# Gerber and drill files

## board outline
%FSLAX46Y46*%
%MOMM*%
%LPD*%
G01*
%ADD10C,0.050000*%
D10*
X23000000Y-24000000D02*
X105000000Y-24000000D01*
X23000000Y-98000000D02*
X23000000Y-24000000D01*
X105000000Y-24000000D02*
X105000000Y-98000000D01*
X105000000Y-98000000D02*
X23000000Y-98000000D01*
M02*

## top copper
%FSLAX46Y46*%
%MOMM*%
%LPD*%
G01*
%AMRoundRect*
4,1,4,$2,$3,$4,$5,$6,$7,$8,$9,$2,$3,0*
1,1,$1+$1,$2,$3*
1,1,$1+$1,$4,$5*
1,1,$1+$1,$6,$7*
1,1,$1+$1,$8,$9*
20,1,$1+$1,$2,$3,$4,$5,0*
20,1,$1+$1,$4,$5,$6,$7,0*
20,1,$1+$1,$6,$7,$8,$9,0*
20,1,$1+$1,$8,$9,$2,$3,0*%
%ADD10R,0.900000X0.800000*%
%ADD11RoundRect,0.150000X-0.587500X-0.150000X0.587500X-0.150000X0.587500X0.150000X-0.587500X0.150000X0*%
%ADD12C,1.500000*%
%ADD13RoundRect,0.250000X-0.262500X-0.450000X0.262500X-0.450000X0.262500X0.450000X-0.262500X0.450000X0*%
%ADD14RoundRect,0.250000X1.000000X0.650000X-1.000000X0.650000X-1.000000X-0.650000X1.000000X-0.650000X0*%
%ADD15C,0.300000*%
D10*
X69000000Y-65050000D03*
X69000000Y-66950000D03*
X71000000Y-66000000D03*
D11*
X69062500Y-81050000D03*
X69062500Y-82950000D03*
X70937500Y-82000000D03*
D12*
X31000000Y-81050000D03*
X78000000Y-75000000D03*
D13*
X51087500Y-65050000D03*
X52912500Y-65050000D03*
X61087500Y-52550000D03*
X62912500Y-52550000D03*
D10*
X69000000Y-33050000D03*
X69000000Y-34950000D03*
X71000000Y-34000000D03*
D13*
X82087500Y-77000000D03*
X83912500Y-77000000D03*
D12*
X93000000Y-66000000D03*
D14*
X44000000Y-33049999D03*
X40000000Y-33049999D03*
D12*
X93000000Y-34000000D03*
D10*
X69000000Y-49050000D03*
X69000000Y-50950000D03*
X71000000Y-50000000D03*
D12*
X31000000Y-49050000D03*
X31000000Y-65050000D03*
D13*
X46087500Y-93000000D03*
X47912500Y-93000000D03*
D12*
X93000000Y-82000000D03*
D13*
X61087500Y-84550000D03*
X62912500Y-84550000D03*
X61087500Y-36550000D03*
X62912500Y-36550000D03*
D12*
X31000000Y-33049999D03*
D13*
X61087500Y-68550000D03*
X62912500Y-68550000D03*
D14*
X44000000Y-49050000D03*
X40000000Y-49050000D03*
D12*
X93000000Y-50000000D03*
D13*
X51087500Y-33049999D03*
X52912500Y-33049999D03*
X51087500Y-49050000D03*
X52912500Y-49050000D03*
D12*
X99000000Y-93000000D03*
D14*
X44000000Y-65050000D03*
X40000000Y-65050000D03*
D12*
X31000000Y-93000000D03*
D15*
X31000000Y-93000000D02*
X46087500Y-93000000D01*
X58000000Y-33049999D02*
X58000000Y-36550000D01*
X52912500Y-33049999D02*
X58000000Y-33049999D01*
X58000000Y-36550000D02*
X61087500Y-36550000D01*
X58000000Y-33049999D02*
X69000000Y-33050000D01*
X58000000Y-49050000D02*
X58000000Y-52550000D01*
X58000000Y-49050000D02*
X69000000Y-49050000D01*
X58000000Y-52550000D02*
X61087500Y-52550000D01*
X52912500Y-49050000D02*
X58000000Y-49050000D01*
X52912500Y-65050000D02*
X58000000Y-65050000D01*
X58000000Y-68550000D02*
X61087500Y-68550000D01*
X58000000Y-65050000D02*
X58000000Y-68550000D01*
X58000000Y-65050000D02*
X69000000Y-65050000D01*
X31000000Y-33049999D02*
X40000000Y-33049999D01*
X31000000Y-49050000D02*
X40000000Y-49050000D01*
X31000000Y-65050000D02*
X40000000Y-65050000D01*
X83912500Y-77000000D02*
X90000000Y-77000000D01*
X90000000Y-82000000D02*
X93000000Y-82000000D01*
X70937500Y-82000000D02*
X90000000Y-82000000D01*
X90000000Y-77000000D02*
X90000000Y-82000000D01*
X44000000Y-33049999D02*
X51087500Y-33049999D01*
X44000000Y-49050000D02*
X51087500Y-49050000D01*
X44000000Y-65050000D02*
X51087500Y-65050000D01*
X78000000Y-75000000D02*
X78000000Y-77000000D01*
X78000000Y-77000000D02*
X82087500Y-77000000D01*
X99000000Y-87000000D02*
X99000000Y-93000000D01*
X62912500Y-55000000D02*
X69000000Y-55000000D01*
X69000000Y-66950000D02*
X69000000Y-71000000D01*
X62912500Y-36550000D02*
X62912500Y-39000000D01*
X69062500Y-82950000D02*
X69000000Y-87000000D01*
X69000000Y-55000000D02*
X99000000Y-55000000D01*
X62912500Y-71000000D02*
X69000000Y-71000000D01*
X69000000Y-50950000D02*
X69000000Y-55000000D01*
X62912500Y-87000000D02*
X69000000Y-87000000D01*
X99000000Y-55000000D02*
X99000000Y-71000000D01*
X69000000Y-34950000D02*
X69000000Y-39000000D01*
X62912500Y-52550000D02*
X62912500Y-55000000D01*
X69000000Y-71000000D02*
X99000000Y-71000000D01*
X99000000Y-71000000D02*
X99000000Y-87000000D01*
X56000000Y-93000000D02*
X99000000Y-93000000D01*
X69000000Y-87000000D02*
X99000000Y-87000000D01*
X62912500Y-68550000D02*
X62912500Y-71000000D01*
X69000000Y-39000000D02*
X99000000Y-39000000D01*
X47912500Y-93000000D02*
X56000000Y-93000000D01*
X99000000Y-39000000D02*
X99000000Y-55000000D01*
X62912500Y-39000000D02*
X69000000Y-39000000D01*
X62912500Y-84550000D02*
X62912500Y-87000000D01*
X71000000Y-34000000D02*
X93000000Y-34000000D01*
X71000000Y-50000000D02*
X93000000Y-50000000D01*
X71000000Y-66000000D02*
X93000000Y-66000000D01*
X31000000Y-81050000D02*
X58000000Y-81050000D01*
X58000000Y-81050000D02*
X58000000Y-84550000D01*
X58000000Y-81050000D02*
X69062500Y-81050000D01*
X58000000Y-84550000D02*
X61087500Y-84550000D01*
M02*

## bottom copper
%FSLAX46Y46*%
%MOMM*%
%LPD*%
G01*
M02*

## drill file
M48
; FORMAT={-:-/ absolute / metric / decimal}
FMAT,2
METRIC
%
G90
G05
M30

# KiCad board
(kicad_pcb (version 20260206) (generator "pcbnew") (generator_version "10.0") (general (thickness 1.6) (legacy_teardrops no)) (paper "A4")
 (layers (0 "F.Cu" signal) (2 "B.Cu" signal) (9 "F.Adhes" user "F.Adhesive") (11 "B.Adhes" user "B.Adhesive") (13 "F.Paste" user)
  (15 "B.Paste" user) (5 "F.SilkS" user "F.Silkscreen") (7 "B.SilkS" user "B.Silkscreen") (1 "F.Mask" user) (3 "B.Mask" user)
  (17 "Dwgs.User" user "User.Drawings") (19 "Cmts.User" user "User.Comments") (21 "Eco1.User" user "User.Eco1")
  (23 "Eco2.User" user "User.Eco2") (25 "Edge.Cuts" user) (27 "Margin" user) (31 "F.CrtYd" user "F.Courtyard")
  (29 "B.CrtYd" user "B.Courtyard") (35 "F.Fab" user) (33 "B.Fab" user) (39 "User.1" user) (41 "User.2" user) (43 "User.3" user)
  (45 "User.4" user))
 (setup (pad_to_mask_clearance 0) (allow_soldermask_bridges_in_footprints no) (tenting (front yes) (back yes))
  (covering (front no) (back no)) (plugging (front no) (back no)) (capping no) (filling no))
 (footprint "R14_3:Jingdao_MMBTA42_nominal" (layer "F.Cu") (at 70 66)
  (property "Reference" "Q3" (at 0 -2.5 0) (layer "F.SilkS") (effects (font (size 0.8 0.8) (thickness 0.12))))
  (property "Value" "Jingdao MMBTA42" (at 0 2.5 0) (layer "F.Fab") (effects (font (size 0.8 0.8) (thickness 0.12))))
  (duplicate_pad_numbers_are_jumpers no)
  (pad "1" smd rect (at -1 -0.95) (size 0.9 0.8) (layers "F.Cu" "F.Mask" "F.Paste") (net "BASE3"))
  (pad "2" smd rect (at -1 0.95) (size 0.9 0.8) (layers "F.Cu" "F.Mask" "F.Paste") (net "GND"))
  (pad "3" smd rect (at 1 0) (size 0.9 0.8) (layers "F.Cu" "F.Mask" "F.Paste") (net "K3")))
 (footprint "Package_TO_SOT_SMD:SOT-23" (layer "F.Cu") (at 70 82)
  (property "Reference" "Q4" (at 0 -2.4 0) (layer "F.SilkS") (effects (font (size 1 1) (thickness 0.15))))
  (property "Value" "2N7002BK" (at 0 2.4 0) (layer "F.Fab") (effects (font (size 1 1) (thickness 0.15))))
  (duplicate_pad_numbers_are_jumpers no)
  (pad "1" smd roundrect (at -0.9375 -0.95) (size 1.475 0.6) (layers "F.Cu" "F.Mask" "F.Paste") (roundrect_rratio 0.25) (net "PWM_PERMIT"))
  (pad "2" smd roundrect (at -0.9375 0.95) (size 1.475 0.6) (layers "F.Cu" "F.Mask" "F.Paste") (roundrect_rratio 0.25) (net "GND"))
  (pad "3" smd roundrect (at 0.9375 0) (size 1.475 0.6) (layers "F.Cu" "F.Mask" "F.Paste") (roundrect_rratio 0.25) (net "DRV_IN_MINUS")))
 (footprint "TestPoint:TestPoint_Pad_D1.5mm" (layer "F.Cu") (at 31 81.05)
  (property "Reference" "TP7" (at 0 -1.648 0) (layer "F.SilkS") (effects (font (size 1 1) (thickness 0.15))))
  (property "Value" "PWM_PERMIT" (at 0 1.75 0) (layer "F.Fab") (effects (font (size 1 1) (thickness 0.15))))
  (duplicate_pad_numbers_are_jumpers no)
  (pad "1" smd circle (at 0 0) (size 1.5 1.5) (layers "F.Cu" "F.Mask") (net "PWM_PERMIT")))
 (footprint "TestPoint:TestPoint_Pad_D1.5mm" (layer "F.Cu") (at 78 75)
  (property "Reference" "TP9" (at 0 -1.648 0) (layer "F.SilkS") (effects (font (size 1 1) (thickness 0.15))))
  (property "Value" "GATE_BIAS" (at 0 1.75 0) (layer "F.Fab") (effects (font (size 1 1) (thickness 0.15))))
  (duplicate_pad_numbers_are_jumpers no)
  (pad "1" smd circle (at 0 0) (size 1.5 1.5) (layers "F.Cu" "F.Mask") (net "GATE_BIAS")))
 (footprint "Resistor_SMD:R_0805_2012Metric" (layer "F.Cu") (at 52 65.05)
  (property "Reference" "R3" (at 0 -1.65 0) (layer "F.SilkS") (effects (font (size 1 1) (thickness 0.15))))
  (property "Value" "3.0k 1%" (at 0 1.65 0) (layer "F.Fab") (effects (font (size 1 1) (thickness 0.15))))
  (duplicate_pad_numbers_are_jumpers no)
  (pad "1" smd roundrect (at -0.9125 0) (size 1.025 1.4) (layers "F.Cu" "F.Mask" "F.Paste") (roundrect_rratio 0.243902) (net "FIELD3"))
  (pad "2" smd roundrect (at 0.9125 0) (size 1.025 1.4) (layers "F.Cu" "F.Mask" "F.Paste") (roundrect_rratio 0.243902) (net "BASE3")))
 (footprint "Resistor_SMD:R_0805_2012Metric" (layer "F.Cu") (at 62 52.55)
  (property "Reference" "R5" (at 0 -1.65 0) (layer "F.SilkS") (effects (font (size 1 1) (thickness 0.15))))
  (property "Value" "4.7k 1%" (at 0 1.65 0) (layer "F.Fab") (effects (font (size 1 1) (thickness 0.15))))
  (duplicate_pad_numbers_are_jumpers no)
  (pad "1" smd roundrect (at -0.9125 0) (size 1.025 1.4) (layers "F.Cu" "F.Mask" "F.Paste") (roundrect_rratio 0.243902) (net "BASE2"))
  (pad "2" smd roundrect (at 0.9125 0) (size 1.025 1.4) (layers "F.Cu" "F.Mask" "F.Paste") (roundrect_rratio 0.243902) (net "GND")))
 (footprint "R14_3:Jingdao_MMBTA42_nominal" (layer "F.Cu") (at 70 34)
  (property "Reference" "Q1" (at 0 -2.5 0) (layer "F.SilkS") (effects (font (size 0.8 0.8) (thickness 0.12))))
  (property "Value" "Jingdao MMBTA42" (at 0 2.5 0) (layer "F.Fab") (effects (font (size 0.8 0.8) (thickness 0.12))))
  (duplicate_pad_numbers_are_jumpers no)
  (pad "1" smd rect (at -1 -0.95) (size 0.9 0.8) (layers "F.Cu" "F.Mask" "F.Paste") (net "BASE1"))
  (pad "2" smd rect (at -1 0.95) (size 0.9 0.8) (layers "F.Cu" "F.Mask" "F.Paste") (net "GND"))
  (pad "3" smd rect (at 1 0) (size 0.9 0.8) (layers "F.Cu" "F.Mask" "F.Paste") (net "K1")))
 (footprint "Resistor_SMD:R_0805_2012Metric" (layer "F.Cu") (at 83 77)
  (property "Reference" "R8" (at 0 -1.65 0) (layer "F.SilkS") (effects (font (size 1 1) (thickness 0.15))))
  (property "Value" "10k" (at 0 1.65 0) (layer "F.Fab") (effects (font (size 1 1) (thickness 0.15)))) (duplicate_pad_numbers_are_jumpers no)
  (pad "1" smd roundrect (at -0.9125 0) (size 1.025 1.4) (layers "F.Cu" "F.Mask" "F.Paste") (roundrect_rratio 0.243902) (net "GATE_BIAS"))
  (pad "2" smd roundrect (at 0.9125 0) (size 1.025 1.4) (layers "F.Cu" "F.Mask" "F.Paste") (roundrect_rratio 0.243902) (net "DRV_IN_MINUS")))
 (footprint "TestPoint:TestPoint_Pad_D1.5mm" (layer "F.Cu") (at 93 66)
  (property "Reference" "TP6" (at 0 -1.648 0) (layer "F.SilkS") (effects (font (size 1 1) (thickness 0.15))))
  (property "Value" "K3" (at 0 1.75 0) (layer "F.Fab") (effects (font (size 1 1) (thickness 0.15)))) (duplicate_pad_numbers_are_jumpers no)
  (pad "1" smd circle (at 0 0) (size 1.5 1.5) (layers "F.Cu" "F.Mask") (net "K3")))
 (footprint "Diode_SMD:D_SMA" (layer "F.Cu") (at 42 33.049999 180)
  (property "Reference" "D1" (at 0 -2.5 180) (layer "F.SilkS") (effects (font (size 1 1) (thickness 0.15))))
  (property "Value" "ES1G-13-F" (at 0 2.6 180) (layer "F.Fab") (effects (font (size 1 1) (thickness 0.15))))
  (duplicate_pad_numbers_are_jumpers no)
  (pad "1" smd roundrect (at -2 0 180) (size 2.5 1.8) (layers "F.Cu" "F.Mask" "F.Paste") (roundrect_rratio 0.1388888889) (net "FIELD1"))
  (pad "2" smd roundrect (at 2 0 180) (size 2.5 1.8) (layers "F.Cu" "F.Mask" "F.Paste") (roundrect_rratio 0.1388888889) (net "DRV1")))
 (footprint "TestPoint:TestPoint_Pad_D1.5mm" (layer "F.Cu") (at 93 34)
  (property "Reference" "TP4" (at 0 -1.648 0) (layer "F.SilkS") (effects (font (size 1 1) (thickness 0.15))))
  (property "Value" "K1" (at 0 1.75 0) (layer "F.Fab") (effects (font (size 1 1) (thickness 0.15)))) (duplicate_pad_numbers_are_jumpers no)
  (pad "1" smd circle (at 0 0) (size 1.5 1.5) (layers "F.Cu" "F.Mask") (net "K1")))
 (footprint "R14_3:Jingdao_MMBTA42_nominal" (layer "F.Cu") (at 70 50)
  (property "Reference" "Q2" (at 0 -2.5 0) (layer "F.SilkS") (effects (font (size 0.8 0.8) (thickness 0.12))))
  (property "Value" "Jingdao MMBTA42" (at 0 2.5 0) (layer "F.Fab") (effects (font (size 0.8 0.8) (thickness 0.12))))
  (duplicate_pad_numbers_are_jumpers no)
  (pad "1" smd rect (at -1 -0.95) (size 0.9 0.8) (layers "F.Cu" "F.Mask" "F.Paste") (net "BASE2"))
  (pad "2" smd rect (at -1 0.95) (size 0.9 0.8) (layers "F.Cu" "F.Mask" "F.Paste") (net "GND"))
  (pad "3" smd rect (at 1 0) (size 0.9 0.8) (layers "F.Cu" "F.Mask" "F.Paste") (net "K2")))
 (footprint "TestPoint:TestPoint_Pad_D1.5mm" (layer "F.Cu") (at 31 49.05)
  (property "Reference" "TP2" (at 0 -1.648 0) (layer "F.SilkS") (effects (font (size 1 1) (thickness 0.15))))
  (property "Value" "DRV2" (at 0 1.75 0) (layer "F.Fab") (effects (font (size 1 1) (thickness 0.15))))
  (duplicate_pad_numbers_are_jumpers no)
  (pad "1" smd circle (at 0 0) (size 1.5 1.5) (layers "F.Cu" "F.Mask") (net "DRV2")))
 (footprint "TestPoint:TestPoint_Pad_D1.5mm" (layer "F.Cu") (at 31 65.05)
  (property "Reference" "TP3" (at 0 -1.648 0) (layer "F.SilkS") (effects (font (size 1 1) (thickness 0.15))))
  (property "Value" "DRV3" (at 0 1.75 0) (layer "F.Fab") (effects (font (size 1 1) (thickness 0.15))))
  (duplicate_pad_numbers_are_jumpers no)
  (pad "1" smd circle (at 0 0) (size 1.5 1.5) (layers "F.Cu" "F.Mask") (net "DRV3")))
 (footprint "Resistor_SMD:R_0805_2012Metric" (layer "F.Cu") (at 47 93)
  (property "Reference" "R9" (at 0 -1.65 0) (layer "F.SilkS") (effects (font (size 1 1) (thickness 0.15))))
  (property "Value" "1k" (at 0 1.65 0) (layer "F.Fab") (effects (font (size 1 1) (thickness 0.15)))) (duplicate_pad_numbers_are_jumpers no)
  (pad "1" smd roundrect (at -0.9125 0) (size 1.025 1.4) (layers "F.Cu" "F.Mask" "F.Paste") (roundrect_rratio 0.243902) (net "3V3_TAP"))
  (pad "2" smd roundrect (at 0.9125 0) (size 1.025 1.4) (layers "F.Cu" "F.Mask" "F.Paste") (roundrect_rratio 0.243902) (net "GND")))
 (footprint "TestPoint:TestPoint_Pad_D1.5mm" (layer "F.Cu") (at 93 82)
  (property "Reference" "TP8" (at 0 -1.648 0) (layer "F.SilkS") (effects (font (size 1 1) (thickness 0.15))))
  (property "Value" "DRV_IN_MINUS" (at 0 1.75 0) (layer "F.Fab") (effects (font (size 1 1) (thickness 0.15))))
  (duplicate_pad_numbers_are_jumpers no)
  (pad "1" smd circle (at 0 0) (size 1.5 1.5) (layers "F.Cu" "F.Mask") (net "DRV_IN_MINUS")))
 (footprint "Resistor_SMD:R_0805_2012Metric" (layer "F.Cu") (at 62 84.55)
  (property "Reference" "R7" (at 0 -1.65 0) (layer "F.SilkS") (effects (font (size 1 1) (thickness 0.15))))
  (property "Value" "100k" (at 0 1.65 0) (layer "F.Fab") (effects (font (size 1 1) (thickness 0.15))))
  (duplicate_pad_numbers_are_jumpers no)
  (pad "1" smd roundrect (at -0.9125 0) (size 1.025 1.4) (layers "F.Cu" "F.Mask" "F.Paste") (roundrect_rratio 0.243902) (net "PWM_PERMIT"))
  (pad "2" smd roundrect (at 0.9125 0) (size 1.025 1.4) (layers "F.Cu" "F.Mask" "F.Paste") (roundrect_rratio 0.243902) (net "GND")))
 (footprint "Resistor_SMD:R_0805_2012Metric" (layer "F.Cu") (at 62 36.55)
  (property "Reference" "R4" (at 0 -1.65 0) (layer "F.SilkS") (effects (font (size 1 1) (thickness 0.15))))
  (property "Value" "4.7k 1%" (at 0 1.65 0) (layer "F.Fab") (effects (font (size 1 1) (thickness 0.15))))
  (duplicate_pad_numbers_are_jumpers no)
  (pad "1" smd roundrect (at -0.9125 0) (size 1.025 1.4) (layers "F.Cu" "F.Mask" "F.Paste") (roundrect_rratio 0.243902) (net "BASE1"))
  (pad "2" smd roundrect (at 0.9125 0) (size 1.025 1.4) (layers "F.Cu" "F.Mask" "F.Paste") (roundrect_rratio 0.243902) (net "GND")))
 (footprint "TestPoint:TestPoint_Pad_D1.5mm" (layer "F.Cu") (at 31 33.049999)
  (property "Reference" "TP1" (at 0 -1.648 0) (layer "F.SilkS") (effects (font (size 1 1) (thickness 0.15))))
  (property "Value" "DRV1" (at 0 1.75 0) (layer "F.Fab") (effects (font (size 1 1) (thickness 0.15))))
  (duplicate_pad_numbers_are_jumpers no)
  (pad "1" smd circle (at 0 0) (size 1.5 1.5) (layers "F.Cu" "F.Mask") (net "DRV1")))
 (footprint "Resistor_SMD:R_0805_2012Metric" (layer "F.Cu") (at 62 68.55)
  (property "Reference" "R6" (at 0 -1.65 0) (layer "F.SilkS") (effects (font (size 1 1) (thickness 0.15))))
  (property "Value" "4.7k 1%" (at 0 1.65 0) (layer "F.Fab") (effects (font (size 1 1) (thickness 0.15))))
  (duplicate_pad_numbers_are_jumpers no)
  (pad "1" smd roundrect (at -0.9125 0) (size 1.025 1.4) (layers "F.Cu" "F.Mask" "F.Paste") (roundrect_rratio 0.243902) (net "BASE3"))
  (pad "2" smd roundrect (at 0.9125 0) (size 1.025 1.4) (layers "F.Cu" "F.Mask" "F.Paste") (roundrect_rratio 0.243902) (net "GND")))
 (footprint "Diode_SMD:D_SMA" (layer "F.Cu") (at 42 49.05 180)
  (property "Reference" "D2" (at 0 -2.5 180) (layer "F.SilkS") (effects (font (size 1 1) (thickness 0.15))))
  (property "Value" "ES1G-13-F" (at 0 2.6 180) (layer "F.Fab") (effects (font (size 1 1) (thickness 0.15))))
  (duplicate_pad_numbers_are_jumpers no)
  (pad "1" smd roundrect (at -2 0 180) (size 2.5 1.8) (layers "F.Cu" "F.Mask" "F.Paste") (roundrect_rratio 0.1388888889) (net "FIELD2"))
  (pad "2" smd roundrect (at 2 0 180) (size 2.5 1.8) (layers "F.Cu" "F.Mask" "F.Paste") (roundrect_rratio 0.1388888889) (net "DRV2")))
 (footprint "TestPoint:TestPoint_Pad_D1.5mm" (layer "F.Cu") (at 93 50)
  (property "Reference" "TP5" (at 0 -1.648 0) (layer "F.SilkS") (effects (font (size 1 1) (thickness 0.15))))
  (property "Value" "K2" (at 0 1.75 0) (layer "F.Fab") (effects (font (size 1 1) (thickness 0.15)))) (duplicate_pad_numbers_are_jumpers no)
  (pad "1" smd circle (at 0 0) (size 1.5 1.5) (layers "F.Cu" "F.Mask") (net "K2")))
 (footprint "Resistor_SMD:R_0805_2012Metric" (layer "F.Cu") (at 52 33.049999)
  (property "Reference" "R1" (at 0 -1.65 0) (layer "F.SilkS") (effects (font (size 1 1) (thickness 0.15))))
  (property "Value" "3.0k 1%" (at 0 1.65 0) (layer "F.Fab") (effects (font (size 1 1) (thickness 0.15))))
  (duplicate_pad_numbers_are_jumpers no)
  (pad "1" smd roundrect (at -0.9125 0) (size 1.025 1.4) (layers "F.Cu" "F.Mask" "F.Paste") (roundrect_rratio 0.243902) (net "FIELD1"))
  (pad "2" smd roundrect (at 0.9125 0) (size 1.025 1.4) (layers "F.Cu" "F.Mask" "F.Paste") (roundrect_rratio 0.243902) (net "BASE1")))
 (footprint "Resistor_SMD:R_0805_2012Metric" (layer "F.Cu") (at 52 49.05)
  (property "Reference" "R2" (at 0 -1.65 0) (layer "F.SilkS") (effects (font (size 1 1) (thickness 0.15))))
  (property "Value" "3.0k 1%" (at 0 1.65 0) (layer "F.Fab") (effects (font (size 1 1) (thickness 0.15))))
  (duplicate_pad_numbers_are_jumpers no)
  (pad "1" smd roundrect (at -0.9125 0) (size 1.025 1.4) (layers "F.Cu" "F.Mask" "F.Paste") (roundrect_rratio 0.243902) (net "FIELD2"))
  (pad "2" smd roundrect (at 0.9125 0) (size 1.025 1.4) (layers "F.Cu" "F.Mask" "F.Paste") (roundrect_rratio 0.243902) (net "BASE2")))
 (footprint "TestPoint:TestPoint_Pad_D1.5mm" (layer "F.Cu") (at 99 93)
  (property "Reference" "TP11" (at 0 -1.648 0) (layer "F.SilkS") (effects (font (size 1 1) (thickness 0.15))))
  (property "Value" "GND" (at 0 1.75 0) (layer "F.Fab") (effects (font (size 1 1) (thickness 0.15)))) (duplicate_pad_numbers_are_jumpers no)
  (pad "1" smd circle (at 0 0) (size 1.5 1.5) (layers "F.Cu" "F.Mask") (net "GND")))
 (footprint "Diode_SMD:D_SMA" (layer "F.Cu") (at 42 65.05 180)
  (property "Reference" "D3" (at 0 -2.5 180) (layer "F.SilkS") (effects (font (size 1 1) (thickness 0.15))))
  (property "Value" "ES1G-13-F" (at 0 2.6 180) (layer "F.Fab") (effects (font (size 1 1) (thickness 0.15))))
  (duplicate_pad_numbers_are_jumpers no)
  (pad "1" smd roundrect (at -2 0 180) (size 2.5 1.8) (layers "F.Cu" "F.Mask" "F.Paste") (roundrect_rratio 0.1388888889) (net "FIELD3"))
  (pad "2" smd roundrect (at 2 0 180) (size 2.5 1.8) (layers "F.Cu" "F.Mask" "F.Paste") (roundrect_rratio 0.1388888889) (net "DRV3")))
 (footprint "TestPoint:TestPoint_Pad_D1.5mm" (layer "F.Cu") (at 31 93)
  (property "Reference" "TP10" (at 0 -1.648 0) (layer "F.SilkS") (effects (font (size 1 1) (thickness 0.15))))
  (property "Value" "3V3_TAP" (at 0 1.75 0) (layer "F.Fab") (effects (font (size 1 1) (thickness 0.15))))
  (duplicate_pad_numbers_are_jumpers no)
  (pad "1" smd circle (at 0 0) (size 1.5 1.5) (layers "F.Cu" "F.Mask") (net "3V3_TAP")))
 (gr_line (start 23 24) (end 105 24) (stroke (width 0.05) (type default)) (layer "Edge.Cuts"))
 (gr_line (start 23 98) (end 23 24) (stroke (width 0.05) (type default)) (layer "Edge.Cuts"))
 (gr_line (start 105 24) (end 105 98) (stroke (width 0.05) (type default)) (layer "Edge.Cuts"))
 (gr_line (start 105 98) (end 23 98) (stroke (width 0.05) (type default)) (layer "Edge.Cuts"))
 (segment (start 31 93) (end 46.0875 93) (width 0.3) (layer "F.Cu") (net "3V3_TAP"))
 (segment (start 58 33.049999) (end 58 36.55) (width 0.3) (layer "F.Cu") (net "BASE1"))
 (segment (start 52.9125 33.049999) (end 58 33.049999) (width 0.3) (layer "F.Cu") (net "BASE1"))
 (segment (start 58 36.55) (end 61.0875 36.55) (width 0.3) (layer "F.Cu") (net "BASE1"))
 (segment (start 58 33.049999) (end 69 33.05) (width 0.3) (layer "F.Cu") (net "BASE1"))
 (segment (start 58 49.05) (end 58 52.55) (width 0.3) (layer "F.Cu") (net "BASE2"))
 (segment (start 58 49.05) (end 69 49.05) (width 0.3) (layer "F.Cu") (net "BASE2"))
 (segment (start 58 52.55) (end 61.0875 52.55) (width 0.3) (layer "F.Cu") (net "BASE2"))
 (segment (start 52.9125 49.05) (end 58 49.05) (width 0.3) (layer "F.Cu") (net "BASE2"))
 (segment (start 52.9125 65.05) (end 58 65.05) (width 0.3) (layer "F.Cu") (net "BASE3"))
 (segment (start 58 68.55) (end 61.0875 68.55) (width 0.3) (layer "F.Cu") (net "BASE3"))
 (segment (start 58 65.05) (end 58 68.55) (width 0.3) (layer "F.Cu") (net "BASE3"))
 (segment (start 58 65.05) (end 69 65.05) (width 0.3) (layer "F.Cu") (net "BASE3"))
 (segment (start 31 33.049999) (end 40 33.049999) (width 0.3) (layer "F.Cu") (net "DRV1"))
 (segment (start 31 49.05) (end 40 49.05) (width 0.3) (layer "F.Cu") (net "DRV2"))
 (segment (start 31 65.05) (end 40 65.05) (width 0.3) (layer "F.Cu") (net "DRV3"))
 (segment (start 83.9125 77) (end 90 77) (width 0.3) (layer "F.Cu") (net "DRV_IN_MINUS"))
 (segment (start 90 82) (end 93 82) (width 0.3) (layer "F.Cu") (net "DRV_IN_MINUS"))
 (segment (start 70.9375 82) (end 90 82) (width 0.3) (layer "F.Cu") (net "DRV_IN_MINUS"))
 (segment (start 90 77) (end 90 82) (width 0.3) (layer "F.Cu") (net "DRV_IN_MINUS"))
 (segment (start 44 33.049999) (end 51.0875 33.049999) (width 0.3) (layer "F.Cu") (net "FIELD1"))
 (segment (start 44 49.05) (end 51.0875 49.05) (width 0.3) (layer "F.Cu") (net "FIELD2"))
 (segment (start 44 65.05) (end 51.0875 65.05) (width 0.3) (layer "F.Cu") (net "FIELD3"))
 (segment (start 78 75) (end 78 77) (width 0.3) (layer "F.Cu") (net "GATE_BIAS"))
 (segment (start 78 77) (end 82.0875 77) (width 0.3) (layer "F.Cu") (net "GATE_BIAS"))
 (segment (start 99 87) (end 99 93) (width 0.3) (layer "F.Cu") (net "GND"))
 (segment (start 62.9125 55) (end 69 55) (width 0.3) (layer "F.Cu") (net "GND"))
 (segment (start 69 66.95) (end 69 71) (width 0.3) (layer "F.Cu") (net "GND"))
 (segment (start 62.9125 36.55) (end 62.9125 39) (width 0.3) (layer "F.Cu") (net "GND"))
 (segment (start 69.0625 82.95) (end 69 87) (width 0.3) (layer "F.Cu") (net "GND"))
 (segment (start 69 55) (end 99 55) (width 0.3) (layer "F.Cu") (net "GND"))
 (segment (start 62.9125 71) (end 69 71) (width 0.3) (layer "F.Cu") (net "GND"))
 (segment (start 69 50.95) (end 69 55) (width 0.3) (layer "F.Cu") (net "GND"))
 (segment (start 62.9125 87) (end 69 87) (width 0.3) (layer "F.Cu") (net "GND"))
 (segment (start 99 55) (end 99 71) (width 0.3) (layer "F.Cu") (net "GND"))
 (segment (start 69 34.95) (end 69 39) (width 0.3) (layer "F.Cu") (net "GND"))
 (segment (start 62.9125 52.55) (end 62.9125 55) (width 0.3) (layer "F.Cu") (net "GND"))
 (segment (start 69 71) (end 99 71) (width 0.3) (layer "F.Cu") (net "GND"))
 (segment (start 99 71) (end 99 87) (width 0.3) (layer "F.Cu") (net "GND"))
 (segment (start 56 93) (end 99 93) (width 0.3) (layer "F.Cu") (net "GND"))
 (segment (start 69 87) (end 99 87) (width 0.3) (layer "F.Cu") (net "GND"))
 (segment (start 62.9125 68.55) (end 62.9125 71) (width 0.3) (layer "F.Cu") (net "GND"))
 (segment (start 69 39) (end 99 39) (width 0.3) (layer "F.Cu") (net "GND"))
 (segment (start 47.9125 93) (end 56 93) (width 0.3) (layer "F.Cu") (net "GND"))
 (segment (start 99 39) (end 99 55) (width 0.3) (layer "F.Cu") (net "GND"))
 (segment (start 62.9125 39) (end 69 39) (width 0.3) (layer "F.Cu") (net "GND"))
 (segment (start 62.9125 84.55) (end 62.9125 87) (width 0.3) (layer "F.Cu") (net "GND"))
 (segment (start 71 34) (end 93 34) (width 0.3) (layer "F.Cu") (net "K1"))
 (segment (start 71 50) (end 93 50) (width 0.3) (layer "F.Cu") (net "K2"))
 (segment (start 71 66) (end 93 66) (width 0.3) (layer "F.Cu") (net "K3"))
 (segment (start 31 81.05) (end 58 81.05) (width 0.3) (layer "F.Cu") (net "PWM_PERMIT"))
 (segment (start 58 81.05) (end 58 84.55) (width 0.3) (layer "F.Cu") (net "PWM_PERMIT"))
 (segment (start 58 81.05) (end 69.0625 81.05) (width 0.3) (layer "F.Cu") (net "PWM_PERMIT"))
 (segment (start 58 84.55) (end 61.0875 84.55) (width 0.3) (layer "F.Cu") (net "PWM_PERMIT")))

